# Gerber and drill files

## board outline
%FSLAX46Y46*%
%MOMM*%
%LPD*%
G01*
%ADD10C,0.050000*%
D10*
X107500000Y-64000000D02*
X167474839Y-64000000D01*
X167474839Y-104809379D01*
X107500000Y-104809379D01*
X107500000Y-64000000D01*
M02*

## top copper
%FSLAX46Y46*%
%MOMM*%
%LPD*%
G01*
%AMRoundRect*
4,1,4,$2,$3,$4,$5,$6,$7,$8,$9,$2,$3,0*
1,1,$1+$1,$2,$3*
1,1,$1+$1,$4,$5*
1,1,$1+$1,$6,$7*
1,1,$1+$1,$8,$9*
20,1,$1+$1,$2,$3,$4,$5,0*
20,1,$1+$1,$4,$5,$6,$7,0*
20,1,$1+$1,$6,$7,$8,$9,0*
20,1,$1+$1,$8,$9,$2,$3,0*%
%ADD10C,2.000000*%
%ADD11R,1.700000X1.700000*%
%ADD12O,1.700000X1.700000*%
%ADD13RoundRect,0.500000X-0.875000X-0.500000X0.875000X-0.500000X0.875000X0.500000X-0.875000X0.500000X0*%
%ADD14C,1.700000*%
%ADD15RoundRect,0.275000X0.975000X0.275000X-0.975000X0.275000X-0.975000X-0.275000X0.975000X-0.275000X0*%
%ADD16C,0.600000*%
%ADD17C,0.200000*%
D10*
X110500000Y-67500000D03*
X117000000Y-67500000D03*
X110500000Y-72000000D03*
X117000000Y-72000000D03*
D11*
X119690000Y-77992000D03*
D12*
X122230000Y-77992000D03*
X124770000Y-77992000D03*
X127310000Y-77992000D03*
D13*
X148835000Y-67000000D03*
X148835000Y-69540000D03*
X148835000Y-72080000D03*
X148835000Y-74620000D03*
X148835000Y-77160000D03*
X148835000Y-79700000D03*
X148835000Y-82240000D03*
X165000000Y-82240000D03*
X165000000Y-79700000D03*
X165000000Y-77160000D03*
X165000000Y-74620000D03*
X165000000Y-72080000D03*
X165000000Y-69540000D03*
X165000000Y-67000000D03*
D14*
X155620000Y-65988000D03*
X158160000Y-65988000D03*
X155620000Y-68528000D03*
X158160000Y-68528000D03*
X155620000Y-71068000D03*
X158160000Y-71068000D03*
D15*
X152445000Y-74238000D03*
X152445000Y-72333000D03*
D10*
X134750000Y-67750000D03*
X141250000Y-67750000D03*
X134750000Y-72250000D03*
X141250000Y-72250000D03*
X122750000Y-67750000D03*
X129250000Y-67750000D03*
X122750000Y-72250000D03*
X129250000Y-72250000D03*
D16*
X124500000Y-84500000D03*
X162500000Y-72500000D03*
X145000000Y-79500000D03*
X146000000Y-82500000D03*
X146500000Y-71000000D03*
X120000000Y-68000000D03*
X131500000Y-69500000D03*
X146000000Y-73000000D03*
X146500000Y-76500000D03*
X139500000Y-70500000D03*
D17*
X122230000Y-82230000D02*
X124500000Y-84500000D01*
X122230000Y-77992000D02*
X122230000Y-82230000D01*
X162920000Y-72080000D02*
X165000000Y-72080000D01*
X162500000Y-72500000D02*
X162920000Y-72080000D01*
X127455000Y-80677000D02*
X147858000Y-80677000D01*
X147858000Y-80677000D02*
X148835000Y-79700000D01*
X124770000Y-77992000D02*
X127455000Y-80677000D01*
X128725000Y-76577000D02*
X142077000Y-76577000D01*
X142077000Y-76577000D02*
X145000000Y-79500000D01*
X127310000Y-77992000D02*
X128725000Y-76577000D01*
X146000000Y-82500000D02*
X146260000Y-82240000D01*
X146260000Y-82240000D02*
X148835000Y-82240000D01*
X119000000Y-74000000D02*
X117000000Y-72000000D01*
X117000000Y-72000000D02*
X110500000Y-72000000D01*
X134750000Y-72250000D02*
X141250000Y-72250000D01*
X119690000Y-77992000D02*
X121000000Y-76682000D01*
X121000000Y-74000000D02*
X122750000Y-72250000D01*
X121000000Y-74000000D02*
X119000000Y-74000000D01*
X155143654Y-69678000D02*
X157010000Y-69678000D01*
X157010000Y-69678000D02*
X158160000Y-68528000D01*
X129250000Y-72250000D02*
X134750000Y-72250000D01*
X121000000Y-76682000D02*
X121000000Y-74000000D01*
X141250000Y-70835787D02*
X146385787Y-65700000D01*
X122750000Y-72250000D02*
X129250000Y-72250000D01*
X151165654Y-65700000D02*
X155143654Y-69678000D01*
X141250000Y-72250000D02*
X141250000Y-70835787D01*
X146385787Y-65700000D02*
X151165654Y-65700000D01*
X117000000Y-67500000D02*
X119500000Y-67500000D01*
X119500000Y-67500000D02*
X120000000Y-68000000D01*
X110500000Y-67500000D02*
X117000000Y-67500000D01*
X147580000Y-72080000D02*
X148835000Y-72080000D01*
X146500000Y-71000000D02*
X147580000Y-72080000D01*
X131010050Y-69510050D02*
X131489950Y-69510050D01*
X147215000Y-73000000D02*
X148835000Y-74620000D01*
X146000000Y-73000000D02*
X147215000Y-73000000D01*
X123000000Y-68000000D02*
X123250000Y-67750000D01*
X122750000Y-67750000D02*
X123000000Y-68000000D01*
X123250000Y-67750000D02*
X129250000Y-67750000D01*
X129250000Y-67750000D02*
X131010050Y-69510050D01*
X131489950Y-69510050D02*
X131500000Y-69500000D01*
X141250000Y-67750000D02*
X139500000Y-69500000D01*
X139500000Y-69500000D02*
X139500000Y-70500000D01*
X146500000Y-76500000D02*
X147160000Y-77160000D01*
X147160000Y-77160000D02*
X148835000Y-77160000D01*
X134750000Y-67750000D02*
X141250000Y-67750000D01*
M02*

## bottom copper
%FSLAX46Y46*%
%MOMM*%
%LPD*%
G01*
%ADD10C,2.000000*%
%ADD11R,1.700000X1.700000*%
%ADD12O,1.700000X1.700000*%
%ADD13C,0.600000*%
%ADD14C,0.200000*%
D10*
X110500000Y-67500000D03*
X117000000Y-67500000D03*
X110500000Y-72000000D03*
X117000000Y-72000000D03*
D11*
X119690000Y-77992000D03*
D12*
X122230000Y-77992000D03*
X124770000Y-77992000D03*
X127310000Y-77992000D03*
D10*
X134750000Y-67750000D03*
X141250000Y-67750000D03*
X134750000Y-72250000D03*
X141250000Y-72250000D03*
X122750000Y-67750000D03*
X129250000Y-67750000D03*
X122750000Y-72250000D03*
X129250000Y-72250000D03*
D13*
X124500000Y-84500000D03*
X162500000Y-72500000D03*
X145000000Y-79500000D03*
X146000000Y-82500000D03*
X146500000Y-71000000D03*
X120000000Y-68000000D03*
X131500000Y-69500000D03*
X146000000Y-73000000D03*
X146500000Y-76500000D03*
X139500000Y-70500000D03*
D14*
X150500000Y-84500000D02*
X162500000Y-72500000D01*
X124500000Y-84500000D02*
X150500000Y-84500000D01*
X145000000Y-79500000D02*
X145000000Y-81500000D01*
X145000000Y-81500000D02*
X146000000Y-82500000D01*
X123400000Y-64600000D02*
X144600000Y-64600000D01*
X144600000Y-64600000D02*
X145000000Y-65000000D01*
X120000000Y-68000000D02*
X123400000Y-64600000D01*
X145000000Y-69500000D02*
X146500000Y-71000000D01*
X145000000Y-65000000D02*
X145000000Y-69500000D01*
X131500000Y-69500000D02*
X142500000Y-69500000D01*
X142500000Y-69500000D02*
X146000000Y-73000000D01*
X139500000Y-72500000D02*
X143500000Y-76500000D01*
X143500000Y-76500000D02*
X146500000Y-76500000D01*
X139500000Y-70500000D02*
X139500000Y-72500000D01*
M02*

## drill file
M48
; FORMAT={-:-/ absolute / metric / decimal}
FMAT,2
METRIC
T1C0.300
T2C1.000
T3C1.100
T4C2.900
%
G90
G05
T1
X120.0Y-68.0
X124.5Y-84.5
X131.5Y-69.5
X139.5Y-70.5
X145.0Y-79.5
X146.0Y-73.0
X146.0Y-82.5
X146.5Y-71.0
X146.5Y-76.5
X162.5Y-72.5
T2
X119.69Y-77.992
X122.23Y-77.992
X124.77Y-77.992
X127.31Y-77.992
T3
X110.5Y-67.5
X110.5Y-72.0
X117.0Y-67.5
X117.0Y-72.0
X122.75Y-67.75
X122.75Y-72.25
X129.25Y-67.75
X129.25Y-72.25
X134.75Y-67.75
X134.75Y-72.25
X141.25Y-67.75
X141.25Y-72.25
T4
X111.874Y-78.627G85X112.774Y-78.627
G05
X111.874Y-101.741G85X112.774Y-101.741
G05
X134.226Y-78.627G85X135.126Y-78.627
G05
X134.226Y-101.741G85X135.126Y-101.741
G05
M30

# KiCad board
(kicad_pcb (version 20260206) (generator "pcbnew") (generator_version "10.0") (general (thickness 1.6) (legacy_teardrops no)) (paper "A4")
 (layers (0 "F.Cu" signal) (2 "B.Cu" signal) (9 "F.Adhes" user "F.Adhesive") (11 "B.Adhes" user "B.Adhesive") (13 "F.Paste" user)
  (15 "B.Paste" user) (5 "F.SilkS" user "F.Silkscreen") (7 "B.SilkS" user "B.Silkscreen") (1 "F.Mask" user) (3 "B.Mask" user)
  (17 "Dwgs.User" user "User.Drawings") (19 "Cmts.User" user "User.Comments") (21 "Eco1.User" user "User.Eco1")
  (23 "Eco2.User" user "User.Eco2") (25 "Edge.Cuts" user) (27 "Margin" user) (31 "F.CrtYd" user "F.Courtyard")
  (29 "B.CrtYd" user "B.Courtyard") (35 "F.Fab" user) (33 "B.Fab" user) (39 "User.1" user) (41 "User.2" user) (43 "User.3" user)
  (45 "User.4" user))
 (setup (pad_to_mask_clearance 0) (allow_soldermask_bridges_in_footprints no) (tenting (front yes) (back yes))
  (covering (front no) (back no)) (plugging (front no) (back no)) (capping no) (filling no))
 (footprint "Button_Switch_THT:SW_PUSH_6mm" (layer "F.Cu") (at 110.5 67.5)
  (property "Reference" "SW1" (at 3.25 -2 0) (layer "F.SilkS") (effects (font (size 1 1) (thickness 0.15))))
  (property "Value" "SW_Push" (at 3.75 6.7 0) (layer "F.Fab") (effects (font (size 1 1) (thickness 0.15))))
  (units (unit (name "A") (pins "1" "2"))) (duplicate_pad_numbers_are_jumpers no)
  (pad "1" thru_hole circle (at 0 0 90) (size 2 2) (drill 1.1) (layers "*.Cu" "*.Mask") (remove_unused_layers no) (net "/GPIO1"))
  (pad "1" thru_hole circle (at 6.5 0 90) (size 2 2) (drill 1.1) (layers "*.Cu" "*.Mask") (remove_unused_layers no) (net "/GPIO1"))
  (pad "2" thru_hole circle (at 0 4.5 90) (size 2 2) (drill 1.1) (layers "*.Cu" "*.Mask") (remove_unused_layers no) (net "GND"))
  (pad "2" thru_hole circle (at 6.5 4.5 90) (size 2 2) (drill 1.1) (layers "*.Cu" "*.Mask") (remove_unused_layers no) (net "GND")))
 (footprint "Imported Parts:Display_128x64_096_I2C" (layer "F.Cu") (at 123.5 77.992)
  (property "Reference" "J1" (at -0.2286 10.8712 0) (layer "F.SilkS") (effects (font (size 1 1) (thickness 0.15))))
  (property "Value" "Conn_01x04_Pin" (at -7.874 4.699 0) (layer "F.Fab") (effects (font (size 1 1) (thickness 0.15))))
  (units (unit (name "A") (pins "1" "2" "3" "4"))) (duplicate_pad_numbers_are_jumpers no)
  (pad "" np_thru_hole oval (at -11.176 0.635) (size 3.8 2.9) (drill oval 3.8 2.9) (layers "*.Cu" "*.Mask"))
  (pad "" np_thru_hole oval (at -11.176 23.749) (size 3.8 2.9) (drill oval 3.8 2.9) (layers "*.Cu" "*.Mask"))
  (pad "" np_thru_hole oval (at 11.176 0.635) (size 3.8 2.9) (drill oval 3.8 2.9) (layers "*.Cu" "*.Mask"))
  (pad "" np_thru_hole oval (at 11.176 23.749) (size 3.8 2.9) (drill oval 3.8 2.9) (layers "*.Cu" "*.Mask"))
  (pad "1" thru_hole rect (at -3.81 0 90) (size 1.7 1.7) (drill 1) (layers "*.Cu" "*.Mask") (remove_unused_layers no) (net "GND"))
  (pad "2" thru_hole oval (at -1.27 0 90) (size 1.7 1.7) (drill 1) (layers "*.Cu" "*.Mask") (remove_unused_layers no) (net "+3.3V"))
  (pad "3" thru_hole oval (at 1.27 0 90) (size 1.7 1.7) (drill 1) (layers "*.Cu" "*.Mask") (remove_unused_layers no) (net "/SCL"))
  (pad "4" thru_hole oval (at 3.81 0 90) (size 1.7 1.7) (drill 1) (layers "*.Cu" "*.Mask") (remove_unused_layers no) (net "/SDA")))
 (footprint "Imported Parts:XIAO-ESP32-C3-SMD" (layer "F.Cu") (at 148 85.12)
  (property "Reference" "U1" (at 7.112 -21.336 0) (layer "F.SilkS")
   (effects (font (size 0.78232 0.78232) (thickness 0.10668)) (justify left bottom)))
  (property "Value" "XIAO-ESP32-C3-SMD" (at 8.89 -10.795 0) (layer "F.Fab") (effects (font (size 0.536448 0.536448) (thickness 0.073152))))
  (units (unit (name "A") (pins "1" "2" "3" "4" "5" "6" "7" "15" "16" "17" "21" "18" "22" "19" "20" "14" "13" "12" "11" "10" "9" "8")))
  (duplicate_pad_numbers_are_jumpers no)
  (pad "1" smd roundrect (at 0.835 -18.12) (size 2.75 2) (layers "F.Cu" "F.Mask" "F.Paste") (roundrect_rratio 0.25)
   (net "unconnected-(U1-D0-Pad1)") (solder_mask_margin 0.0508) (thermal_bridge_angle 45))
  (pad "2" smd roundrect (at 0.835 -15.58) (size 2.75 2) (layers "F.Cu" "F.Mask" "F.Paste") (roundrect_rratio 0.25)
   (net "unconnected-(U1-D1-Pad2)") (solder_mask_margin 0.0508) (thermal_bridge_angle 45))
  (pad "3" smd roundrect (at 0.835 -13.04) (size 2.75 2) (layers "F.Cu" "F.Mask" "F.Paste") (roundrect_rratio 0.25) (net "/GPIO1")
   (solder_mask_margin 0.0508) (thermal_bridge_angle 45))
  (pad "4" smd roundrect (at 0.835 -10.5) (size 2.75 2) (layers "F.Cu" "F.Mask" "F.Paste") (roundrect_rratio 0.25) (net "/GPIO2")
   (solder_mask_margin 0.0508) (thermal_bridge_angle 45))
  (pad "5" smd roundrect (at 0.835 -7.96) (size 2.75 2) (layers "F.Cu" "F.Mask" "F.Paste") (roundrect_rratio 0.25) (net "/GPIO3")
   (solder_mask_margin 0.0508) (thermal_bridge_angle 45))
  (pad "6" smd roundrect (at 0.835 -5.42) (size 2.75 2) (layers "F.Cu" "F.Mask" "F.Paste") (roundrect_rratio 0.25) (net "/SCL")
   (solder_mask_margin 0.0508) (thermal_bridge_angle 45))
  (pad "7" smd roundrect (at 0.835 -2.88) (size 2.75 2) (layers "F.Cu" "F.Mask" "F.Paste") (roundrect_rratio 0.25) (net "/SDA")
   (solder_mask_margin 0.0508) (thermal_bridge_angle 45))
  (pad "8" smd roundrect (at 17 -2.88) (size 2.75 2) (layers "F.Cu" "F.Mask" "F.Paste") (roundrect_rratio 0.25)
   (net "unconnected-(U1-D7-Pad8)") (solder_mask_margin 0.0508) (thermal_bridge_angle 45))
  (pad "9" smd roundrect (at 17 -5.42) (size 2.75 2) (layers "F.Cu" "F.Mask" "F.Paste") (roundrect_rratio 0.25)
   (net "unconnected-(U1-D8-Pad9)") (solder_mask_margin 0.0508) (thermal_bridge_angle 45))
  (pad "10" smd roundrect (at 17 -7.96) (size 2.75 2) (layers "F.Cu" "F.Mask" "F.Paste") (roundrect_rratio 0.25)
   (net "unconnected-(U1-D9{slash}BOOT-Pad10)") (solder_mask_margin 0.0508) (thermal_bridge_angle 45))
  (pad "11" smd roundrect (at 17 -10.5) (size 2.75 2) (layers "F.Cu" "F.Mask" "F.Paste") (roundrect_rratio 0.25)
   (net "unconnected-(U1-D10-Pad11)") (solder_mask_margin 0.0508) (thermal_bridge_angle 45))
  (pad "12" smd roundrect (at 17 -13.04) (size 2.75 2) (layers "F.Cu" "F.Mask" "F.Paste") (roundrect_rratio 0.25) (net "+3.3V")
   (solder_mask_margin 0.0508) (thermal_bridge_angle 45))
  (pad "13" smd roundrect (at 17 -15.58) (size 2.75 2) (layers "F.Cu" "F.Mask" "F.Paste") (roundrect_rratio 0.25) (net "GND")
   (solder_mask_margin 0.0508) (thermal_bridge_angle 45))
  (pad "14" smd roundrect (at 17 -18.12) (size 2.75 2) (layers "F.Cu" "F.Mask" "F.Paste") (roundrect_rratio 0.25) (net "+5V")
   (solder_mask_margin 0.0508) (thermal_bridge_angle 45))
  (pad "15" smd circle (at 7.62 -19.132) (size 1.7 1.7) (layers "F.Cu" "F.Mask" "F.Paste") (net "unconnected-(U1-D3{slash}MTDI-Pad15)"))
  (pad "16" smd circle (at 10.16 -19.132) (size 1.7 1.7) (layers "F.Cu" "F.Mask" "F.Paste") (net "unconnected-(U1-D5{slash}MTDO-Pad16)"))
  (pad "17" smd circle (at 7.62 -16.592) (size 1.7 1.7) (layers "F.Cu" "F.Mask" "F.Paste") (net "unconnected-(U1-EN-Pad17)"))
  (pad "18" smd circle (at 10.16 -16.592) (size 1.7 1.7) (layers "F.Cu" "F.Mask" "F.Paste") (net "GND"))
  (pad "19" smd circle (at 7.62 -14.052) (size 1.7 1.7) (layers "F.Cu" "F.Mask" "F.Paste") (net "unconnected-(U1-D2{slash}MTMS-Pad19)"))
  (pad "20" smd circle (at 10.16 -14.052) (size 1.7 1.7) (layers "F.Cu" "F.Mask" "F.Paste") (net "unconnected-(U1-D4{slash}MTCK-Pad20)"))
  (pad "21" smd roundrect (at 4.445 -10.882 180) (size 2.5 1.1) (layers "F.Cu" "F.Mask" "F.Paste") (roundrect_rratio 0.25)
   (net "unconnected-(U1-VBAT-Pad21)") (thermal_bridge_angle 45))
  (pad "22" smd roundrect (at 4.445 -12.787 180) (size 2.5 1.1) (layers "F.Cu" "F.Mask" "F.Paste") (roundrect_rratio 0.25)
   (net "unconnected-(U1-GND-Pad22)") (thermal_bridge_angle 45)))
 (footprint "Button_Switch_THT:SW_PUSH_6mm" (layer "F.Cu") (at 134.75 67.75)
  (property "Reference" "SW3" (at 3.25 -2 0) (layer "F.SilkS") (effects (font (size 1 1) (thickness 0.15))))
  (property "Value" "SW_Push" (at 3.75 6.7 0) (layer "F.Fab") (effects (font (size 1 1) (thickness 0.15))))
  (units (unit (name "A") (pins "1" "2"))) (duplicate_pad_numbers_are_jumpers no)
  (pad "1" thru_hole circle (at 0 0 90) (size 2 2) (drill 1.1) (layers "*.Cu" "*.Mask") (remove_unused_layers no) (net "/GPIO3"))
  (pad "1" thru_hole circle (at 6.5 0 90) (size 2 2) (drill 1.1) (layers "*.Cu" "*.Mask") (remove_unused_layers no) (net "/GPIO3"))
  (pad "2" thru_hole circle (at 0 4.5 90) (size 2 2) (drill 1.1) (layers "*.Cu" "*.Mask") (remove_unused_layers no) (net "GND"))
  (pad "2" thru_hole circle (at 6.5 4.5 90) (size 2 2) (drill 1.1) (layers "*.Cu" "*.Mask") (remove_unused_layers no) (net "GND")))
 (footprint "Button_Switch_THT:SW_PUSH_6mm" (layer "F.Cu") (at 122.75 67.75)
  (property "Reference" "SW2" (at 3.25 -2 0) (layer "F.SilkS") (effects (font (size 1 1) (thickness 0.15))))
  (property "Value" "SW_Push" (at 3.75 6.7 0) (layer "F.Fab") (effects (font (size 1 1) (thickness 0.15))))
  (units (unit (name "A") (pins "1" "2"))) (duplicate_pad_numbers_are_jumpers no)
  (pad "1" thru_hole circle (at 0 0 90) (size 2 2) (drill 1.1) (layers "*.Cu" "*.Mask") (remove_unused_layers no) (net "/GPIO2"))
  (pad "1" thru_hole circle (at 6.5 0 90) (size 2 2) (drill 1.1) (layers "*.Cu" "*.Mask") (remove_unused_layers no) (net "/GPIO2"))
  (pad "2" thru_hole circle (at 0 4.5 90) (size 2 2) (drill 1.1) (layers "*.Cu" "*.Mask") (remove_unused_layers no) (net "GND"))
  (pad "2" thru_hole circle (at 6.5 4.5 90) (size 2 2) (drill 1.1) (layers "*.Cu" "*.Mask") (remove_unused_layers no) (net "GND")))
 (gr_rect (start 107.5 64) (end 167.474839 104.809379) (stroke (width 0.05) (type default)) (fill no) (layer "Edge.Cuts"))
 (segment (start 122.23 82.23) (end 124.5 84.5) (width 0.2) (layer "F.Cu") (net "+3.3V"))
 (segment (start 122.23 77.992) (end 122.23 82.23) (width 0.2) (layer "F.Cu") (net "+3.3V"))
 (segment (start 162.92 72.08) (end 165 72.08) (width 0.2) (layer "F.Cu") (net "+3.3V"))
 (segment (start 162.5 72.5) (end 162.92 72.08) (width 0.2) (layer "F.Cu") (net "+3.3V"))
 (via (at 124.5 84.5) (size 0.6) (drill 0.3) (layers "F.Cu" "B.Cu") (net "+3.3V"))
 (via (at 162.5 72.5) (size 0.6) (drill 0.3) (layers "F.Cu" "B.Cu") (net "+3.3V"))
 (segment (start 150.5 84.5) (end 162.5 72.5) (width 0.2) (layer "B.Cu") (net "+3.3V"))
 (segment (start 124.5 84.5) (end 150.5 84.5) (width 0.2) (layer "B.Cu") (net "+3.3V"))
 (segment (start 127.455 80.677) (end 147.858 80.677) (width 0.2) (layer "F.Cu") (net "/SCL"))
 (segment (start 147.858 80.677) (end 148.835 79.7) (width 0.2) (layer "F.Cu") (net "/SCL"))
 (segment (start 124.77 77.992) (end 127.455 80.677) (width 0.2) (layer "F.Cu") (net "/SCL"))
 (segment (start 128.725 76.577) (end 142.077 76.577) (width 0.2) (layer "F.Cu") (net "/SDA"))
 (segment (start 142.077 76.577) (end 145 79.5) (width 0.2) (layer "F.Cu") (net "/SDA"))
 (segment (start 127.31 77.992) (end 128.725 76.577) (width 0.2) (layer "F.Cu") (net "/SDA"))
 (segment (start 146 82.5) (end 146.26 82.24) (width 0.2) (layer "F.Cu") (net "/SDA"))
 (segment (start 146.26 82.24) (end 148.835 82.24) (width 0.2) (layer "F.Cu") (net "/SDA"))
 (via (at 145 79.5) (size 0.6) (drill 0.3) (layers "F.Cu" "B.Cu") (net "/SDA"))
 (via (at 146 82.5) (size 0.6) (drill 0.3) (layers "F.Cu" "B.Cu") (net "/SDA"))
 (segment (start 145 79.5) (end 145 81.5) (width 0.2) (layer "B.Cu") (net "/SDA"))
 (segment (start 145 81.5) (end 146 82.5) (width 0.2) (layer "B.Cu") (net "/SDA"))
 (segment (start 119 74) (end 117 72) (width 0.2) (layer "F.Cu") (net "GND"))
 (segment (start 117 72) (end 110.5 72) (width 0.2) (layer "F.Cu") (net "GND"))
 (segment (start 134.75 72.25) (end 141.25 72.25) (width 0.2) (layer "F.Cu") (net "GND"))
 (segment (start 119.69 77.992) (end 121 76.682) (width 0.2) (layer "F.Cu") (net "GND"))
 (segment (start 121 74) (end 122.75 72.25) (width 0.2) (layer "F.Cu") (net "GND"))
 (segment (start 121 74) (end 119 74) (width 0.2) (layer "F.Cu") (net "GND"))
 (segment (start 155.143654 69.678) (end 157.01 69.678) (width 0.2) (layer "F.Cu") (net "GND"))
 (segment (start 157.01 69.678) (end 158.16 68.528) (width 0.2) (layer "F.Cu") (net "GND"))
 (segment (start 129.25 72.25) (end 134.75 72.25) (width 0.2) (layer "F.Cu") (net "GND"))
 (segment (start 121 76.682) (end 121 74) (width 0.2) (layer "F.Cu") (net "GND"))
 (segment (start 141.25 70.835787) (end 146.385787 65.7) (width 0.2) (layer "F.Cu") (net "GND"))
 (segment (start 122.75 72.25) (end 129.25 72.25) (width 0.2) (layer "F.Cu") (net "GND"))
 (segment (start 151.165654 65.7) (end 155.143654 69.678) (width 0.2) (layer "F.Cu") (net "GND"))
 (segment (start 141.25 72.25) (end 141.25 70.835787) (width 0.2) (layer "F.Cu") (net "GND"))
 (segment (start 146.385787 65.7) (end 151.165654 65.7) (width 0.2) (layer "F.Cu") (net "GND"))
 (segment (start 117 67.5) (end 119.5 67.5) (width 0.2) (layer "F.Cu") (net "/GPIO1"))
 (segment (start 119.5 67.5) (end 120 68) (width 0.2) (layer "F.Cu") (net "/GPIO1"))
 (segment (start 110.5 67.5) (end 117 67.5) (width 0.2) (layer "F.Cu") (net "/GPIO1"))
 (segment (start 147.58 72.08) (end 148.835 72.08) (width 0.2) (layer "F.Cu") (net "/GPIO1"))
 (segment (start 146.5 71) (end 147.58 72.08) (width 0.2) (layer "F.Cu") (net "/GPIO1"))
 (via (at 146.5 71) (size 0.6) (drill 0.3) (layers "F.Cu" "B.Cu") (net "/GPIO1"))
 (via (at 120 68) (size 0.6) (drill 0.3) (layers "F.Cu" "B.Cu") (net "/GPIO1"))
 (segment (start 123.4 64.6) (end 144.6 64.6) (width 0.2) (layer "B.Cu") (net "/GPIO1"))
 (segment (start 144.6 64.6) (end 145 65) (width 0.2) (layer "B.Cu") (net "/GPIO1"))
 (segment (start 120 68) (end 123.4 64.6) (width 0.2) (layer "B.Cu") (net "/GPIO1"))
 (segment (start 145 69.5) (end 146.5 71) (width 0.2) (layer "B.Cu") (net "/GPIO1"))
 (segment (start 145 65) (end 145 69.5) (width 0.2) (layer "B.Cu") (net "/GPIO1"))
 (segment (start 131.01005 69.51005) (end 131.48995 69.51005) (width 0.2) (layer "F.Cu") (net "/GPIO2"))
 (segment (start 147.215 73) (end 148.835 74.62) (width 0.2) (layer "F.Cu") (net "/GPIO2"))
 (segment (start 146 73) (end 147.215 73) (width 0.2) (layer "F.Cu") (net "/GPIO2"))
 (segment (start 123 68) (end 123.25 67.75) (width 0.2) (layer "F.Cu") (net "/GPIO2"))
 (segment (start 122.75 67.75) (end 123 68) (width 0.2) (layer "F.Cu") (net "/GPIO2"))
 (segment (start 123.25 67.75) (end 129.25 67.75) (width 0.2) (layer "F.Cu") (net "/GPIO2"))
 (segment (start 129.25 67.75) (end 131.01005 69.51005) (width 0.2) (layer "F.Cu") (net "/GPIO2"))
 (segment (start 131.48995 69.51005) (end 131.5 69.5) (width 0.2) (layer "F.Cu") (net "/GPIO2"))
 (via (at 131.5 69.5) (size 0.6) (drill 0.3) (layers "F.Cu" "B.Cu") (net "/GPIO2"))
 (via (at 146 73) (size 0.6) (drill 0.3) (layers "F.Cu" "B.Cu") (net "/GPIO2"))
 (segment (start 131.5 69.5) (end 142.5 69.5) (width 0.2) (layer "B.Cu") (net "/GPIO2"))
 (segment (start 142.5 69.5) (end 146 73) (width 0.2) (layer "B.Cu") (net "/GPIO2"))
 (segment (start 141.25 67.75) (end 139.5 69.5) (width 0.2) (layer "F.Cu") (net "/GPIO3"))
 (segment (start 139.5 69.5) (end 139.5 70.5) (width 0.2) (layer "F.Cu") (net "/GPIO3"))
 (segment (start 146.5 76.5) (end 147.16 77.16) (width 0.2) (layer "F.Cu") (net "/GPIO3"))
 (segment (start 147.16 77.16) (end 148.835 77.16) (width 0.2) (layer "F.Cu") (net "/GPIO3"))
 (segment (start 134.75 67.75) (end 141.25 67.75) (width 0.2) (layer "F.Cu") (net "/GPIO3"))
 (via (at 146.5 76.5) (size 0.6) (drill 0.3) (layers "F.Cu" "B.Cu") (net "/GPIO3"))
 (via (at 139.5 70.5) (size 0.6) (drill 0.3) (layers "F.Cu" "B.Cu") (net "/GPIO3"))
 (segment (start 139.5 72.5) (end 143.5 76.5) (width 0.2) (layer "B.Cu") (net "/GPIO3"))
 (segment (start 143.5 76.5) (end 146.5 76.5) (width 0.2) (layer "B.Cu") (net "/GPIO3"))
 (segment (start 139.5 70.5) (end 139.5 72.5) (width 0.2) (layer "B.Cu") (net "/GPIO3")))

